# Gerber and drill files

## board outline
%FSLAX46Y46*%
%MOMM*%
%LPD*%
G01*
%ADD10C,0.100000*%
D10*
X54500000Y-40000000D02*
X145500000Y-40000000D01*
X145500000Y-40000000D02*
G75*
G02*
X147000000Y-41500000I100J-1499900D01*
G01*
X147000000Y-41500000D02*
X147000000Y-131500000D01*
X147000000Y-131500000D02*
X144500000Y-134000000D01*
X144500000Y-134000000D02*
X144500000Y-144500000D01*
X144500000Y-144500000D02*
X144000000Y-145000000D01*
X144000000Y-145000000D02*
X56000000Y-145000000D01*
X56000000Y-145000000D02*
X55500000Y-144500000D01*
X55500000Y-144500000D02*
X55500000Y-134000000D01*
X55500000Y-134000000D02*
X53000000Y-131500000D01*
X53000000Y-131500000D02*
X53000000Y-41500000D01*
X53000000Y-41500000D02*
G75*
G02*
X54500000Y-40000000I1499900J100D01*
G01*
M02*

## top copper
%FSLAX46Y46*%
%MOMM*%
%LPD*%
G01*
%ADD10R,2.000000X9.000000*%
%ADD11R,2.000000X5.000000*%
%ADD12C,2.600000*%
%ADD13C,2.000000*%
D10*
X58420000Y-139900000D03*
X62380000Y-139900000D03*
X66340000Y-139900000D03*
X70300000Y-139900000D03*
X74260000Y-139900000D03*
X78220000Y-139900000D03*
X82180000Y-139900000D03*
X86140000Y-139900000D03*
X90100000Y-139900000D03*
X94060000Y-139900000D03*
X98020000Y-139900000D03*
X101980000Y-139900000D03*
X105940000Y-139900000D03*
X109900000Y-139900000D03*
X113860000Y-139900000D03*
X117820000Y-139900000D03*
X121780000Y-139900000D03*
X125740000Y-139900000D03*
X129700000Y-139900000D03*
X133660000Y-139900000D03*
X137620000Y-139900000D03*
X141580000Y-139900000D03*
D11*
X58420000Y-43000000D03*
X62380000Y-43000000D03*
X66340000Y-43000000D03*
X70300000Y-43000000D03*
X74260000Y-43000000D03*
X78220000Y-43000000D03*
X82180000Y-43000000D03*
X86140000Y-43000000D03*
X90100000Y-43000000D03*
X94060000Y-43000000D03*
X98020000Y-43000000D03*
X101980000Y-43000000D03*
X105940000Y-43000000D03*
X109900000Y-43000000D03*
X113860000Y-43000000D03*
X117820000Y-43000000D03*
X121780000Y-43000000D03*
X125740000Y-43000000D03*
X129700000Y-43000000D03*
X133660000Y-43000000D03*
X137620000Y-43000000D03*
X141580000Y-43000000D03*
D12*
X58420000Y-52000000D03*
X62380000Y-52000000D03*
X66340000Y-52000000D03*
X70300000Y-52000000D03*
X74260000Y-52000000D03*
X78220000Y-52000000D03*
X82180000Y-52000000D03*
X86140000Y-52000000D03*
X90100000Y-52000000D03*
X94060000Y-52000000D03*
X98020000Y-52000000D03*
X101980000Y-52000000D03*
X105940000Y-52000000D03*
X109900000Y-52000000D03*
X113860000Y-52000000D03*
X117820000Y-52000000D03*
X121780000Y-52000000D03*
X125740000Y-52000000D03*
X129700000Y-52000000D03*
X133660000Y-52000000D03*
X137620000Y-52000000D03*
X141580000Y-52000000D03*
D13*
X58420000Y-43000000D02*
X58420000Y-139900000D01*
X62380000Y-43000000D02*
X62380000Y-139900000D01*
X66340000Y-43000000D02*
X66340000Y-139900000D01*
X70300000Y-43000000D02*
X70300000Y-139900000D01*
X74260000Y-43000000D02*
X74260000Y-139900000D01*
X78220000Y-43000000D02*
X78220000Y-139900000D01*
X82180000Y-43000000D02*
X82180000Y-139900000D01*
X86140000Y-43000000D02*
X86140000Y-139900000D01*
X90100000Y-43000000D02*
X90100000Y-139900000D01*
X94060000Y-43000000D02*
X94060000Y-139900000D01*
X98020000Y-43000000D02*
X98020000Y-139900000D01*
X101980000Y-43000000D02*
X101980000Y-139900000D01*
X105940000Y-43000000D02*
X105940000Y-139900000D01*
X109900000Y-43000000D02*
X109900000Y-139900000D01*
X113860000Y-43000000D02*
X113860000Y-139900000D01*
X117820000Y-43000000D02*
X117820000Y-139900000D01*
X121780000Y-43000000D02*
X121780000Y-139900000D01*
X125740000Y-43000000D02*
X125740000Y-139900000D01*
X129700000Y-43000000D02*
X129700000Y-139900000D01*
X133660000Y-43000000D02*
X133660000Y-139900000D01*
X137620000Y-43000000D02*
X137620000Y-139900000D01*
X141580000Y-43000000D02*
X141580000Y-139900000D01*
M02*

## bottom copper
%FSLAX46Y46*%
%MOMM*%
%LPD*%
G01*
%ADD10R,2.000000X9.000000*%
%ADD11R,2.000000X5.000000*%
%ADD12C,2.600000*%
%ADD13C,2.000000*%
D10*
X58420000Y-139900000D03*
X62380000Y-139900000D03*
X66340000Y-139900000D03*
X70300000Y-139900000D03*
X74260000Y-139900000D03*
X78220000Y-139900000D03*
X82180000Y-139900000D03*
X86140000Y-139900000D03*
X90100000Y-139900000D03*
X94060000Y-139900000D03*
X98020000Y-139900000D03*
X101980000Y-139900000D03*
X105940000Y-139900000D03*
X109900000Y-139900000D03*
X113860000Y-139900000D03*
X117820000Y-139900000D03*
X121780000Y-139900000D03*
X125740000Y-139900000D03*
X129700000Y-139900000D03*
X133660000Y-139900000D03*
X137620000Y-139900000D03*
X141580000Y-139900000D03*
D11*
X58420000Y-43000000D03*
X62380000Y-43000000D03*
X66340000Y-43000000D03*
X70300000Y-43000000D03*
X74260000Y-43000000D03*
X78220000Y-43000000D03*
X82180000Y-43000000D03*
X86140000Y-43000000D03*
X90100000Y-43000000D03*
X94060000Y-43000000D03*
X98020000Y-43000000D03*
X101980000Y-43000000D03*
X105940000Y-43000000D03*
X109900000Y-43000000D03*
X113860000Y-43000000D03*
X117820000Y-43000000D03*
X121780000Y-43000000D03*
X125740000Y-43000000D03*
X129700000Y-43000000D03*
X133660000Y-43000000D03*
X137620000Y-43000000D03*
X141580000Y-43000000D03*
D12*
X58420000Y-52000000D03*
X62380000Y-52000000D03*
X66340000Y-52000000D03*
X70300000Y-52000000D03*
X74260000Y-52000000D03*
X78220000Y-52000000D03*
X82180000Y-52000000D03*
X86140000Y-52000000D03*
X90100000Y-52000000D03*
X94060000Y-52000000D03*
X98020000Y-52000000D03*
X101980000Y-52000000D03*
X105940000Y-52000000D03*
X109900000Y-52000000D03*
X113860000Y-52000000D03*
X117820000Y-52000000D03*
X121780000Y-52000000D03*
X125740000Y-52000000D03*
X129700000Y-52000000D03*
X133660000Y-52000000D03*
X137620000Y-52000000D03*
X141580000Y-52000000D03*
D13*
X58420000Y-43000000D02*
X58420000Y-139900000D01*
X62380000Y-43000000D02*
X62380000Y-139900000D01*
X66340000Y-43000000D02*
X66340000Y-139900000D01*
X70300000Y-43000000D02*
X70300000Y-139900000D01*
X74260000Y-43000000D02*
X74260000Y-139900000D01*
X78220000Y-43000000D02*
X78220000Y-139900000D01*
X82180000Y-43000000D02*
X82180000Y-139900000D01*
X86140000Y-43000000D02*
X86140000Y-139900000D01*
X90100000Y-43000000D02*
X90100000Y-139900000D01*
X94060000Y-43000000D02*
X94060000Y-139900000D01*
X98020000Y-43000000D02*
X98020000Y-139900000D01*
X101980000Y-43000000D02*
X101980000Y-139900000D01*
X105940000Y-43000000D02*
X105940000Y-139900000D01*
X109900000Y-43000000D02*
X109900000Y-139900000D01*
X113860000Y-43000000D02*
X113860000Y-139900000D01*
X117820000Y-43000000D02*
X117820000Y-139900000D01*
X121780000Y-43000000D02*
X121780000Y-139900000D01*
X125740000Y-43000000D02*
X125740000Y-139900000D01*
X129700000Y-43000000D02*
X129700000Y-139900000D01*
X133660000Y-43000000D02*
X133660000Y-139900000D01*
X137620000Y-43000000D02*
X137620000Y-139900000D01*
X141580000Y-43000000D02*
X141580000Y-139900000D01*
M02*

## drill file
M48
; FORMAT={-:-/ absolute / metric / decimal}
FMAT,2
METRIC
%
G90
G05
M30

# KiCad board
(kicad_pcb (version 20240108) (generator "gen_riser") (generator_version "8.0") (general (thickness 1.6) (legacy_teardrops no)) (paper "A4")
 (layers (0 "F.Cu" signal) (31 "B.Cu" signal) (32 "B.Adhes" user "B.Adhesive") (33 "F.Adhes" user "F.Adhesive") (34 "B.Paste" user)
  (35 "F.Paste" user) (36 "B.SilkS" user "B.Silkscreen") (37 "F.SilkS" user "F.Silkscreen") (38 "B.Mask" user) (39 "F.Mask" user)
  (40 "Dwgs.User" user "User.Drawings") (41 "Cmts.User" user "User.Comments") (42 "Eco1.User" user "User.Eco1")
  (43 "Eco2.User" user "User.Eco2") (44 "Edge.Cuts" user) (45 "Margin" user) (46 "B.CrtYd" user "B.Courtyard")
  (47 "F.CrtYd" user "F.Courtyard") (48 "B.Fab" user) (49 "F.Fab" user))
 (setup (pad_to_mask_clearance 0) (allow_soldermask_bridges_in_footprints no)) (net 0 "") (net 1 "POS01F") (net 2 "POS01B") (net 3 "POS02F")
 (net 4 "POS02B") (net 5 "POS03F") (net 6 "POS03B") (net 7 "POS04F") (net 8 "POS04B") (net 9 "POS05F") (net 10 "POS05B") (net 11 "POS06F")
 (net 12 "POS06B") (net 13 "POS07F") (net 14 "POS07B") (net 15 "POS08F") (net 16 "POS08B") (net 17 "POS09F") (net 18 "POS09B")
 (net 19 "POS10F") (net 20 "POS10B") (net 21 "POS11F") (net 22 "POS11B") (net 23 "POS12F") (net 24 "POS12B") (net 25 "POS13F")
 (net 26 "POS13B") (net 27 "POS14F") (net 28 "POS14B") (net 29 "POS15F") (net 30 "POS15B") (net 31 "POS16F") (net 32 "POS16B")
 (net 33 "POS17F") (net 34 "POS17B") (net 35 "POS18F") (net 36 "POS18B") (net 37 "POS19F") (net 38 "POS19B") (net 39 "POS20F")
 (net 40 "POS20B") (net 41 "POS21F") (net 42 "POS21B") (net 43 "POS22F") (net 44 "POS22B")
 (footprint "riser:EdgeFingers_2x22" (layer "F.Cu") (at 100 40)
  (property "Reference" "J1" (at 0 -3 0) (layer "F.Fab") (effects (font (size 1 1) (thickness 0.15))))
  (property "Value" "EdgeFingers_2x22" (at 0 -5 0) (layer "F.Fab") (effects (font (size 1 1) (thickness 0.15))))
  (pad "1" smd rect (at -41.58 99.9) (size 2 9) (layers "F.Cu" "F.Mask") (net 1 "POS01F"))
  (pad "1B" smd rect (at -41.58 99.9) (size 2 9) (layers "B.Cu" "B.Mask") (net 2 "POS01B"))
  (pad "2" smd rect (at -37.62 99.9) (size 2 9) (layers "F.Cu" "F.Mask") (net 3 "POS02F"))
  (pad "2B" smd rect (at -37.62 99.9) (size 2 9) (layers "B.Cu" "B.Mask") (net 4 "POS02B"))
  (pad "3" smd rect (at -33.66 99.9) (size 2 9) (layers "F.Cu" "F.Mask") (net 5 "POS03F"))
  (pad "3B" smd rect (at -33.66 99.9) (size 2 9) (layers "B.Cu" "B.Mask") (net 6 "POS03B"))
  (pad "4" smd rect (at -29.7 99.9) (size 2 9) (layers "F.Cu" "F.Mask") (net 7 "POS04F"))
  (pad "4B" smd rect (at -29.7 99.9) (size 2 9) (layers "B.Cu" "B.Mask") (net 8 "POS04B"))
  (pad "5" smd rect (at -25.74 99.9) (size 2 9) (layers "F.Cu" "F.Mask") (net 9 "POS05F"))
  (pad "5B" smd rect (at -25.74 99.9) (size 2 9) (layers "B.Cu" "B.Mask") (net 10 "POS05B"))
  (pad "6" smd rect (at -21.78 99.9) (size 2 9) (layers "F.Cu" "F.Mask") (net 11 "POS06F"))
  (pad "6B" smd rect (at -21.78 99.9) (size 2 9) (layers "B.Cu" "B.Mask") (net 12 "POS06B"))
  (pad "7" smd rect (at -17.82 99.9) (size 2 9) (layers "F.Cu" "F.Mask") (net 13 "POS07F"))
  (pad "7B" smd rect (at -17.82 99.9) (size 2 9) (layers "B.Cu" "B.Mask") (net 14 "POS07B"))
  (pad "8" smd rect (at -13.86 99.9) (size 2 9) (layers "F.Cu" "F.Mask") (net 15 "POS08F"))
  (pad "8B" smd rect (at -13.86 99.9) (size 2 9) (layers "B.Cu" "B.Mask") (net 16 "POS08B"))
  (pad "9" smd rect (at -9.9 99.9) (size 2 9) (layers "F.Cu" "F.Mask") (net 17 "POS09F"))
  (pad "9B" smd rect (at -9.9 99.9) (size 2 9) (layers "B.Cu" "B.Mask") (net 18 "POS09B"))
  (pad "10" smd rect (at -5.94 99.9) (size 2 9) (layers "F.Cu" "F.Mask") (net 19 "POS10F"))
  (pad "10B" smd rect (at -5.94 99.9) (size 2 9) (layers "B.Cu" "B.Mask") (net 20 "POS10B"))
  (pad "11" smd rect (at -1.98 99.9) (size 2 9) (layers "F.Cu" "F.Mask") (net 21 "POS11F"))
  (pad "11B" smd rect (at -1.98 99.9) (size 2 9) (layers "B.Cu" "B.Mask") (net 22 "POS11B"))
  (pad "12" smd rect (at 1.98 99.9) (size 2 9) (layers "F.Cu" "F.Mask") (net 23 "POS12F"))
  (pad "12B" smd rect (at 1.98 99.9) (size 2 9) (layers "B.Cu" "B.Mask") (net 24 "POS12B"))
  (pad "13" smd rect (at 5.94 99.9) (size 2 9) (layers "F.Cu" "F.Mask") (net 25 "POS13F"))
  (pad "13B" smd rect (at 5.94 99.9) (size 2 9) (layers "B.Cu" "B.Mask") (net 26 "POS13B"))
  (pad "14" smd rect (at 9.9 99.9) (size 2 9) (layers "F.Cu" "F.Mask") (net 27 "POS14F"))
  (pad "14B" smd rect (at 9.9 99.9) (size 2 9) (layers "B.Cu" "B.Mask") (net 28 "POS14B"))
  (pad "15" smd rect (at 13.86 99.9) (size 2 9) (layers "F.Cu" "F.Mask") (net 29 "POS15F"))
  (pad "15B" smd rect (at 13.86 99.9) (size 2 9) (layers "B.Cu" "B.Mask") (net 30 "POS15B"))
  (pad "16" smd rect (at 17.82 99.9) (size 2 9) (layers "F.Cu" "F.Mask") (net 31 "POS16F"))
  (pad "16B" smd rect (at 17.82 99.9) (size 2 9) (layers "B.Cu" "B.Mask") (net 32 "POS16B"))
  (pad "17" smd rect (at 21.78 99.9) (size 2 9) (layers "F.Cu" "F.Mask") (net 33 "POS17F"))
  (pad "17B" smd rect (at 21.78 99.9) (size 2 9) (layers "B.Cu" "B.Mask") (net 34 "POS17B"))
  (pad "18" smd rect (at 25.74 99.9) (size 2 9) (layers "F.Cu" "F.Mask") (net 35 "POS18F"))
  (pad "18B" smd rect (at 25.74 99.9) (size 2 9) (layers "B.Cu" "B.Mask") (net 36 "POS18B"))
  (pad "19" smd rect (at 29.7 99.9) (size 2 9) (layers "F.Cu" "F.Mask") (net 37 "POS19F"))
  (pad "19B" smd rect (at 29.7 99.9) (size 2 9) (layers "B.Cu" "B.Mask") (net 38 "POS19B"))
  (pad "20" smd rect (at 33.66 99.9) (size 2 9) (layers "F.Cu" "F.Mask") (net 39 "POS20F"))
  (pad "20B" smd rect (at 33.66 99.9) (size 2 9) (layers "B.Cu" "B.Mask") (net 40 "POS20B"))
  (pad "21" smd rect (at 37.62 99.9) (size 2 9) (layers "F.Cu" "F.Mask") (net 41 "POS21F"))
  (pad "21B" smd rect (at 37.62 99.9) (size 2 9) (layers "B.Cu" "B.Mask") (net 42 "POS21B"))
  (pad "22" smd rect (at 41.58 99.9) (size 2 9) (layers "F.Cu" "F.Mask") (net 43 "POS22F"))
  (pad "22B" smd rect (at 41.58 99.9) (size 2 9) (layers "B.Cu" "B.Mask") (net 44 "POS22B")))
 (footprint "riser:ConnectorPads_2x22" (layer "F.Cu") (at 100 40)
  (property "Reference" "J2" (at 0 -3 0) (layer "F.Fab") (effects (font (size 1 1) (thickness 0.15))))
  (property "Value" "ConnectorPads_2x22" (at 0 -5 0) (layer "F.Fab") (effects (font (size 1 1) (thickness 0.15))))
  (pad "1" smd rect (at -41.58 3) (size 2 5) (layers "F.Cu" "F.Mask") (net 1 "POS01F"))
  (pad "1B" smd rect (at -41.58 3) (size 2 5) (layers "B.Cu" "B.Mask") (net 2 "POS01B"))
  (pad "2" smd rect (at -37.62 3) (size 2 5) (layers "F.Cu" "F.Mask") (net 3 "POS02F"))
  (pad "2B" smd rect (at -37.62 3) (size 2 5) (layers "B.Cu" "B.Mask") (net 4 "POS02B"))
  (pad "3" smd rect (at -33.66 3) (size 2 5) (layers "F.Cu" "F.Mask") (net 5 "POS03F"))
  (pad "3B" smd rect (at -33.66 3) (size 2 5) (layers "B.Cu" "B.Mask") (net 6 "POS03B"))
  (pad "4" smd rect (at -29.7 3) (size 2 5) (layers "F.Cu" "F.Mask") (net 7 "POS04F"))
  (pad "4B" smd rect (at -29.7 3) (size 2 5) (layers "B.Cu" "B.Mask") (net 8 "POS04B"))
  (pad "5" smd rect (at -25.74 3) (size 2 5) (layers "F.Cu" "F.Mask") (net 9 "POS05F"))
  (pad "5B" smd rect (at -25.74 3) (size 2 5) (layers "B.Cu" "B.Mask") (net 10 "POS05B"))
  (pad "6" smd rect (at -21.78 3) (size 2 5) (layers "F.Cu" "F.Mask") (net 11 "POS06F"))
  (pad "6B" smd rect (at -21.78 3) (size 2 5) (layers "B.Cu" "B.Mask") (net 12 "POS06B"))
  (pad "7" smd rect (at -17.82 3) (size 2 5) (layers "F.Cu" "F.Mask") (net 13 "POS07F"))
  (pad "7B" smd rect (at -17.82 3) (size 2 5) (layers "B.Cu" "B.Mask") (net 14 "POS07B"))
  (pad "8" smd rect (at -13.86 3) (size 2 5) (layers "F.Cu" "F.Mask") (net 15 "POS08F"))
  (pad "8B" smd rect (at -13.86 3) (size 2 5) (layers "B.Cu" "B.Mask") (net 16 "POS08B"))
  (pad "9" smd rect (at -9.9 3) (size 2 5) (layers "F.Cu" "F.Mask") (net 17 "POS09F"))
  (pad "9B" smd rect (at -9.9 3) (size 2 5) (layers "B.Cu" "B.Mask") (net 18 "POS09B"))
  (pad "10" smd rect (at -5.94 3) (size 2 5) (layers "F.Cu" "F.Mask") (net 19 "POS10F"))
  (pad "10B" smd rect (at -5.94 3) (size 2 5) (layers "B.Cu" "B.Mask") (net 20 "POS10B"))
  (pad "11" smd rect (at -1.98 3) (size 2 5) (layers "F.Cu" "F.Mask") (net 21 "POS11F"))
  (pad "11B" smd rect (at -1.98 3) (size 2 5) (layers "B.Cu" "B.Mask") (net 22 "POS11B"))
  (pad "12" smd rect (at 1.98 3) (size 2 5) (layers "F.Cu" "F.Mask") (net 23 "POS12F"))
  (pad "12B" smd rect (at 1.98 3) (size 2 5) (layers "B.Cu" "B.Mask") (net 24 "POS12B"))
  (pad "13" smd rect (at 5.94 3) (size 2 5) (layers "F.Cu" "F.Mask") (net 25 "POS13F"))
  (pad "13B" smd rect (at 5.94 3) (size 2 5) (layers "B.Cu" "B.Mask") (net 26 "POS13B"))
  (pad "14" smd rect (at 9.9 3) (size 2 5) (layers "F.Cu" "F.Mask") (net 27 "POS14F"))
  (pad "14B" smd rect (at 9.9 3) (size 2 5) (layers "B.Cu" "B.Mask") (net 28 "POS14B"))
  (pad "15" smd rect (at 13.86 3) (size 2 5) (layers "F.Cu" "F.Mask") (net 29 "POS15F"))
  (pad "15B" smd rect (at 13.86 3) (size 2 5) (layers "B.Cu" "B.Mask") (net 30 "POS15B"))
  (pad "16" smd rect (at 17.82 3) (size 2 5) (layers "F.Cu" "F.Mask") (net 31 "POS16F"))
  (pad "16B" smd rect (at 17.82 3) (size 2 5) (layers "B.Cu" "B.Mask") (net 32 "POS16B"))
  (pad "17" smd rect (at 21.78 3) (size 2 5) (layers "F.Cu" "F.Mask") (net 33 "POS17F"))
  (pad "17B" smd rect (at 21.78 3) (size 2 5) (layers "B.Cu" "B.Mask") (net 34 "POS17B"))
  (pad "18" smd rect (at 25.74 3) (size 2 5) (layers "F.Cu" "F.Mask") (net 35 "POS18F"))
  (pad "18B" smd rect (at 25.74 3) (size 2 5) (layers "B.Cu" "B.Mask") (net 36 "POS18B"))
  (pad "19" smd rect (at 29.7 3) (size 2 5) (layers "F.Cu" "F.Mask") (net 37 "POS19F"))
  (pad "19B" smd rect (at 29.7 3) (size 2 5) (layers "B.Cu" "B.Mask") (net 38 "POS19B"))
  (pad "20" smd rect (at 33.66 3) (size 2 5) (layers "F.Cu" "F.Mask") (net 39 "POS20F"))
  (pad "20B" smd rect (at 33.66 3) (size 2 5) (layers "B.Cu" "B.Mask") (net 40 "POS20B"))
  (pad "21" smd rect (at 37.62 3) (size 2 5) (layers "F.Cu" "F.Mask") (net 41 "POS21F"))
  (pad "21B" smd rect (at 37.62 3) (size 2 5) (layers "B.Cu" "B.Mask") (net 42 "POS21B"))
  (pad "22" smd rect (at 41.58 3) (size 2 5) (layers "F.Cu" "F.Mask") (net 43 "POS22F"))
  (pad "22B" smd rect (at 41.58 3) (size 2 5) (layers "B.Cu" "B.Mask") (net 44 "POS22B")))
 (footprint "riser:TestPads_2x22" (layer "F.Cu") (at 100 40)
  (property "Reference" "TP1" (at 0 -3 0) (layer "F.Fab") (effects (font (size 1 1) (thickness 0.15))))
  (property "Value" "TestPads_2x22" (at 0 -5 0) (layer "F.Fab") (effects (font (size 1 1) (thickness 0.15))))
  (pad "1" smd circle (at -41.58 12) (size 2.6 2.6) (layers "F.Cu" "F.Mask") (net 1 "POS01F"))
  (pad "1B" smd circle (at -41.58 12) (size 2.6 2.6) (layers "B.Cu" "B.Mask") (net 2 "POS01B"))
  (pad "2" smd circle (at -37.62 12) (size 2.6 2.6) (layers "F.Cu" "F.Mask") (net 3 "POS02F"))
  (pad "2B" smd circle (at -37.62 12) (size 2.6 2.6) (layers "B.Cu" "B.Mask") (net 4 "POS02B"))
  (pad "3" smd circle (at -33.66 12) (size 2.6 2.6) (layers "F.Cu" "F.Mask") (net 5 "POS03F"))
  (pad "3B" smd circle (at -33.66 12) (size 2.6 2.6) (layers "B.Cu" "B.Mask") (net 6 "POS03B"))
  (pad "4" smd circle (at -29.7 12) (size 2.6 2.6) (layers "F.Cu" "F.Mask") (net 7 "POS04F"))
  (pad "4B" smd circle (at -29.7 12) (size 2.6 2.6) (layers "B.Cu" "B.Mask") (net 8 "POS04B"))
  (pad "5" smd circle (at -25.74 12) (size 2.6 2.6) (layers "F.Cu" "F.Mask") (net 9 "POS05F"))
  (pad "5B" smd circle (at -25.74 12) (size 2.6 2.6) (layers "B.Cu" "B.Mask") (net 10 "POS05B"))
  (pad "6" smd circle (at -21.78 12) (size 2.6 2.6) (layers "F.Cu" "F.Mask") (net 11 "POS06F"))
  (pad "6B" smd circle (at -21.78 12) (size 2.6 2.6) (layers "B.Cu" "B.Mask") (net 12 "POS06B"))
  (pad "7" smd circle (at -17.82 12) (size 2.6 2.6) (layers "F.Cu" "F.Mask") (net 13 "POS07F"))
  (pad "7B" smd circle (at -17.82 12) (size 2.6 2.6) (layers "B.Cu" "B.Mask") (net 14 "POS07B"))
  (pad "8" smd circle (at -13.86 12) (size 2.6 2.6) (layers "F.Cu" "F.Mask") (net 15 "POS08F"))
  (pad "8B" smd circle (at -13.86 12) (size 2.6 2.6) (layers "B.Cu" "B.Mask") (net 16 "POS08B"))
  (pad "9" smd circle (at -9.9 12) (size 2.6 2.6) (layers "F.Cu" "F.Mask") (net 17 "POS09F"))
  (pad "9B" smd circle (at -9.9 12) (size 2.6 2.6) (layers "B.Cu" "B.Mask") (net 18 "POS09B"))
  (pad "10" smd circle (at -5.94 12) (size 2.6 2.6) (layers "F.Cu" "F.Mask") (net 19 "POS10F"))
  (pad "10B" smd circle (at -5.94 12) (size 2.6 2.6) (layers "B.Cu" "B.Mask") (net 20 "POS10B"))
  (pad "11" smd circle (at -1.98 12) (size 2.6 2.6) (layers "F.Cu" "F.Mask") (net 21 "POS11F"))
  (pad "11B" smd circle (at -1.98 12) (size 2.6 2.6) (layers "B.Cu" "B.Mask") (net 22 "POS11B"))
  (pad "12" smd circle (at 1.98 12) (size 2.6 2.6) (layers "F.Cu" "F.Mask") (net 23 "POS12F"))
  (pad "12B" smd circle (at 1.98 12) (size 2.6 2.6) (layers "B.Cu" "B.Mask") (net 24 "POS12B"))
  (pad "13" smd circle (at 5.94 12) (size 2.6 2.6) (layers "F.Cu" "F.Mask") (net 25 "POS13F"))
  (pad "13B" smd circle (at 5.94 12) (size 2.6 2.6) (layers "B.Cu" "B.Mask") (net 26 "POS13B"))
  (pad "14" smd circle (at 9.9 12) (size 2.6 2.6) (layers "F.Cu" "F.Mask") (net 27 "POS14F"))
  (pad "14B" smd circle (at 9.9 12) (size 2.6 2.6) (layers "B.Cu" "B.Mask") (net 28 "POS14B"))
  (pad "15" smd circle (at 13.86 12) (size 2.6 2.6) (layers "F.Cu" "F.Mask") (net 29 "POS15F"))
  (pad "15B" smd circle (at 13.86 12) (size 2.6 2.6) (layers "B.Cu" "B.Mask") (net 30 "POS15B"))
  (pad "16" smd circle (at 17.82 12) (size 2.6 2.6) (layers "F.Cu" "F.Mask") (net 31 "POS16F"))
  (pad "16B" smd circle (at 17.82 12) (size 2.6 2.6) (layers "B.Cu" "B.Mask") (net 32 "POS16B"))
  (pad "17" smd circle (at 21.78 12) (size 2.6 2.6) (layers "F.Cu" "F.Mask") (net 33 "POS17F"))
  (pad "17B" smd circle (at 21.78 12) (size 2.6 2.6) (layers "B.Cu" "B.Mask") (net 34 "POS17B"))
  (pad "18" smd circle (at 25.74 12) (size 2.6 2.6) (layers "F.Cu" "F.Mask") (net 35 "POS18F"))
  (pad "18B" smd circle (at 25.74 12) (size 2.6 2.6) (layers "B.Cu" "B.Mask") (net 36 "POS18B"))
  (pad "19" smd circle (at 29.7 12) (size 2.6 2.6) (layers "F.Cu" "F.Mask") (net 37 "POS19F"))
  (pad "19B" smd circle (at 29.7 12) (size 2.6 2.6) (layers "B.Cu" "B.Mask") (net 38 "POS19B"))
  (pad "20" smd circle (at 33.66 12) (size 2.6 2.6) (layers "F.Cu" "F.Mask") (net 39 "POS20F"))
  (pad "20B" smd circle (at 33.66 12) (size 2.6 2.6) (layers "B.Cu" "B.Mask") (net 40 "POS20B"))
  (pad "21" smd circle (at 37.62 12) (size 2.6 2.6) (layers "F.Cu" "F.Mask") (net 41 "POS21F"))
  (pad "21B" smd circle (at 37.62 12) (size 2.6 2.6) (layers "B.Cu" "B.Mask") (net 42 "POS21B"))
  (pad "22" smd circle (at 41.58 12) (size 2.6 2.6) (layers "F.Cu" "F.Mask") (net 43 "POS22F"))
  (pad "22B" smd circle (at 41.58 12) (size 2.6 2.6) (layers "B.Cu" "B.Mask") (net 44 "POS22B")))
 (segment (start 58.42 43) (end 58.42 139.9) (width 2) (layer "F.Cu") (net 1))
 (segment (start 58.42 43) (end 58.42 139.9) (width 2) (layer "B.Cu") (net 2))
 (segment (start 62.38 43) (end 62.38 139.9) (width 2) (layer "F.Cu") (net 3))
 (segment (start 62.38 43) (end 62.38 139.9) (width 2) (layer "B.Cu") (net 4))
 (segment (start 66.34 43) (end 66.34 139.9) (width 2) (layer "F.Cu") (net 5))
 (segment (start 66.34 43) (end 66.34 139.9) (width 2) (layer "B.Cu") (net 6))
 (segment (start 70.3 43) (end 70.3 139.9) (width 2) (layer "F.Cu") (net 7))
 (segment (start 70.3 43) (end 70.3 139.9) (width 2) (layer "B.Cu") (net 8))
 (segment (start 74.26 43) (end 74.26 139.9) (width 2) (layer "F.Cu") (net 9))
 (segment (start 74.26 43) (end 74.26 139.9) (width 2) (layer "B.Cu") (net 10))
 (segment (start 78.22 43) (end 78.22 139.9) (width 2) (layer "F.Cu") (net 11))
 (segment (start 78.22 43) (end 78.22 139.9) (width 2) (layer "B.Cu") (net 12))
 (segment (start 82.18 43) (end 82.18 139.9) (width 2) (layer "F.Cu") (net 13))
 (segment (start 82.18 43) (end 82.18 139.9) (width 2) (layer "B.Cu") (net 14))
 (segment (start 86.14 43) (end 86.14 139.9) (width 2) (layer "F.Cu") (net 15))
 (segment (start 86.14 43) (end 86.14 139.9) (width 2) (layer "B.Cu") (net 16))
 (segment (start 90.1 43) (end 90.1 139.9) (width 2) (layer "F.Cu") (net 17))
 (segment (start 90.1 43) (end 90.1 139.9) (width 2) (layer "B.Cu") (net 18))
 (segment (start 94.06 43) (end 94.06 139.9) (width 2) (layer "F.Cu") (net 19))
 (segment (start 94.06 43) (end 94.06 139.9) (width 2) (layer "B.Cu") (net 20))
 (segment (start 98.02 43) (end 98.02 139.9) (width 2) (layer "F.Cu") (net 21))
 (segment (start 98.02 43) (end 98.02 139.9) (width 2) (layer "B.Cu") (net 22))
 (segment (start 101.98 43) (end 101.98 139.9) (width 2) (layer "F.Cu") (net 23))
 (segment (start 101.98 43) (end 101.98 139.9) (width 2) (layer "B.Cu") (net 24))
 (segment (start 105.94 43) (end 105.94 139.9) (width 2) (layer "F.Cu") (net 25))
 (segment (start 105.94 43) (end 105.94 139.9) (width 2) (layer "B.Cu") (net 26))
 (segment (start 109.9 43) (end 109.9 139.9) (width 2) (layer "F.Cu") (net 27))
 (segment (start 109.9 43) (end 109.9 139.9) (width 2) (layer "B.Cu") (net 28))
 (segment (start 113.86 43) (end 113.86 139.9) (width 2) (layer "F.Cu") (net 29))
 (segment (start 113.86 43) (end 113.86 139.9) (width 2) (layer "B.Cu") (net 30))
 (segment (start 117.82 43) (end 117.82 139.9) (width 2) (layer "F.Cu") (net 31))
 (segment (start 117.82 43) (end 117.82 139.9) (width 2) (layer "B.Cu") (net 32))
 (segment (start 121.78 43) (end 121.78 139.9) (width 2) (layer "F.Cu") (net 33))
 (segment (start 121.78 43) (end 121.78 139.9) (width 2) (layer "B.Cu") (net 34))
 (segment (start 125.74 43) (end 125.74 139.9) (width 2) (layer "F.Cu") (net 35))
 (segment (start 125.74 43) (end 125.74 139.9) (width 2) (layer "B.Cu") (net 36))
 (segment (start 129.7 43) (end 129.7 139.9) (width 2) (layer "F.Cu") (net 37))
 (segment (start 129.7 43) (end 129.7 139.9) (width 2) (layer "B.Cu") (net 38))
 (segment (start 133.66 43) (end 133.66 139.9) (width 2) (layer "F.Cu") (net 39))
 (segment (start 133.66 43) (end 133.66 139.9) (width 2) (layer "B.Cu") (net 40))
 (segment (start 137.62 43) (end 137.62 139.9) (width 2) (layer "F.Cu") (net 41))
 (segment (start 137.62 43) (end 137.62 139.9) (width 2) (layer "B.Cu") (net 42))
 (segment (start 141.58 43) (end 141.58 139.9) (width 2) (layer "F.Cu") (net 43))
 (segment (start 141.58 43) (end 141.58 139.9) (width 2) (layer "B.Cu") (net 44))
 (gr_line (start 54.5 40) (end 145.5 40) (stroke (width 0.1) (type default)) (layer "Edge.Cuts"))
 (gr_arc (start 145.5 40) (mid 146.5607 40.4393) (end 147 41.5) (stroke (width 0.1) (type default)) (layer "Edge.Cuts"))
 (gr_line (start 147 41.5) (end 147 131.5) (stroke (width 0.1) (type default)) (layer "Edge.Cuts"))
 (gr_line (start 147 131.5) (end 144.5 134) (stroke (width 0.1) (type default)) (layer "Edge.Cuts"))
 (gr_line (start 144.5 134) (end 144.5 144.5) (stroke (width 0.1) (type default)) (layer "Edge.Cuts"))
 (gr_line (start 144.5 144.5) (end 144 145) (stroke (width 0.1) (type default)) (layer "Edge.Cuts"))
 (gr_line (start 144 145) (end 56 145) (stroke (width 0.1) (type default)) (layer "Edge.Cuts"))
 (gr_line (start 56 145) (end 55.5 144.5) (stroke (width 0.1) (type default)) (layer "Edge.Cuts"))
 (gr_line (start 55.5 144.5) (end 55.5 134) (stroke (width 0.1) (type default)) (layer "Edge.Cuts"))
 (gr_line (start 55.5 134) (end 53 131.5) (stroke (width 0.1) (type default)) (layer "Edge.Cuts"))
 (gr_line (start 53 131.5) (end 53 41.5) (stroke (width 0.1) (type default)) (layer "Edge.Cuts"))
 (gr_arc (start 53 41.5) (mid 53.4393 40.4393) (end 54.5 40) (stroke (width 0.1) (type default)) (layer "Edge.Cuts")))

